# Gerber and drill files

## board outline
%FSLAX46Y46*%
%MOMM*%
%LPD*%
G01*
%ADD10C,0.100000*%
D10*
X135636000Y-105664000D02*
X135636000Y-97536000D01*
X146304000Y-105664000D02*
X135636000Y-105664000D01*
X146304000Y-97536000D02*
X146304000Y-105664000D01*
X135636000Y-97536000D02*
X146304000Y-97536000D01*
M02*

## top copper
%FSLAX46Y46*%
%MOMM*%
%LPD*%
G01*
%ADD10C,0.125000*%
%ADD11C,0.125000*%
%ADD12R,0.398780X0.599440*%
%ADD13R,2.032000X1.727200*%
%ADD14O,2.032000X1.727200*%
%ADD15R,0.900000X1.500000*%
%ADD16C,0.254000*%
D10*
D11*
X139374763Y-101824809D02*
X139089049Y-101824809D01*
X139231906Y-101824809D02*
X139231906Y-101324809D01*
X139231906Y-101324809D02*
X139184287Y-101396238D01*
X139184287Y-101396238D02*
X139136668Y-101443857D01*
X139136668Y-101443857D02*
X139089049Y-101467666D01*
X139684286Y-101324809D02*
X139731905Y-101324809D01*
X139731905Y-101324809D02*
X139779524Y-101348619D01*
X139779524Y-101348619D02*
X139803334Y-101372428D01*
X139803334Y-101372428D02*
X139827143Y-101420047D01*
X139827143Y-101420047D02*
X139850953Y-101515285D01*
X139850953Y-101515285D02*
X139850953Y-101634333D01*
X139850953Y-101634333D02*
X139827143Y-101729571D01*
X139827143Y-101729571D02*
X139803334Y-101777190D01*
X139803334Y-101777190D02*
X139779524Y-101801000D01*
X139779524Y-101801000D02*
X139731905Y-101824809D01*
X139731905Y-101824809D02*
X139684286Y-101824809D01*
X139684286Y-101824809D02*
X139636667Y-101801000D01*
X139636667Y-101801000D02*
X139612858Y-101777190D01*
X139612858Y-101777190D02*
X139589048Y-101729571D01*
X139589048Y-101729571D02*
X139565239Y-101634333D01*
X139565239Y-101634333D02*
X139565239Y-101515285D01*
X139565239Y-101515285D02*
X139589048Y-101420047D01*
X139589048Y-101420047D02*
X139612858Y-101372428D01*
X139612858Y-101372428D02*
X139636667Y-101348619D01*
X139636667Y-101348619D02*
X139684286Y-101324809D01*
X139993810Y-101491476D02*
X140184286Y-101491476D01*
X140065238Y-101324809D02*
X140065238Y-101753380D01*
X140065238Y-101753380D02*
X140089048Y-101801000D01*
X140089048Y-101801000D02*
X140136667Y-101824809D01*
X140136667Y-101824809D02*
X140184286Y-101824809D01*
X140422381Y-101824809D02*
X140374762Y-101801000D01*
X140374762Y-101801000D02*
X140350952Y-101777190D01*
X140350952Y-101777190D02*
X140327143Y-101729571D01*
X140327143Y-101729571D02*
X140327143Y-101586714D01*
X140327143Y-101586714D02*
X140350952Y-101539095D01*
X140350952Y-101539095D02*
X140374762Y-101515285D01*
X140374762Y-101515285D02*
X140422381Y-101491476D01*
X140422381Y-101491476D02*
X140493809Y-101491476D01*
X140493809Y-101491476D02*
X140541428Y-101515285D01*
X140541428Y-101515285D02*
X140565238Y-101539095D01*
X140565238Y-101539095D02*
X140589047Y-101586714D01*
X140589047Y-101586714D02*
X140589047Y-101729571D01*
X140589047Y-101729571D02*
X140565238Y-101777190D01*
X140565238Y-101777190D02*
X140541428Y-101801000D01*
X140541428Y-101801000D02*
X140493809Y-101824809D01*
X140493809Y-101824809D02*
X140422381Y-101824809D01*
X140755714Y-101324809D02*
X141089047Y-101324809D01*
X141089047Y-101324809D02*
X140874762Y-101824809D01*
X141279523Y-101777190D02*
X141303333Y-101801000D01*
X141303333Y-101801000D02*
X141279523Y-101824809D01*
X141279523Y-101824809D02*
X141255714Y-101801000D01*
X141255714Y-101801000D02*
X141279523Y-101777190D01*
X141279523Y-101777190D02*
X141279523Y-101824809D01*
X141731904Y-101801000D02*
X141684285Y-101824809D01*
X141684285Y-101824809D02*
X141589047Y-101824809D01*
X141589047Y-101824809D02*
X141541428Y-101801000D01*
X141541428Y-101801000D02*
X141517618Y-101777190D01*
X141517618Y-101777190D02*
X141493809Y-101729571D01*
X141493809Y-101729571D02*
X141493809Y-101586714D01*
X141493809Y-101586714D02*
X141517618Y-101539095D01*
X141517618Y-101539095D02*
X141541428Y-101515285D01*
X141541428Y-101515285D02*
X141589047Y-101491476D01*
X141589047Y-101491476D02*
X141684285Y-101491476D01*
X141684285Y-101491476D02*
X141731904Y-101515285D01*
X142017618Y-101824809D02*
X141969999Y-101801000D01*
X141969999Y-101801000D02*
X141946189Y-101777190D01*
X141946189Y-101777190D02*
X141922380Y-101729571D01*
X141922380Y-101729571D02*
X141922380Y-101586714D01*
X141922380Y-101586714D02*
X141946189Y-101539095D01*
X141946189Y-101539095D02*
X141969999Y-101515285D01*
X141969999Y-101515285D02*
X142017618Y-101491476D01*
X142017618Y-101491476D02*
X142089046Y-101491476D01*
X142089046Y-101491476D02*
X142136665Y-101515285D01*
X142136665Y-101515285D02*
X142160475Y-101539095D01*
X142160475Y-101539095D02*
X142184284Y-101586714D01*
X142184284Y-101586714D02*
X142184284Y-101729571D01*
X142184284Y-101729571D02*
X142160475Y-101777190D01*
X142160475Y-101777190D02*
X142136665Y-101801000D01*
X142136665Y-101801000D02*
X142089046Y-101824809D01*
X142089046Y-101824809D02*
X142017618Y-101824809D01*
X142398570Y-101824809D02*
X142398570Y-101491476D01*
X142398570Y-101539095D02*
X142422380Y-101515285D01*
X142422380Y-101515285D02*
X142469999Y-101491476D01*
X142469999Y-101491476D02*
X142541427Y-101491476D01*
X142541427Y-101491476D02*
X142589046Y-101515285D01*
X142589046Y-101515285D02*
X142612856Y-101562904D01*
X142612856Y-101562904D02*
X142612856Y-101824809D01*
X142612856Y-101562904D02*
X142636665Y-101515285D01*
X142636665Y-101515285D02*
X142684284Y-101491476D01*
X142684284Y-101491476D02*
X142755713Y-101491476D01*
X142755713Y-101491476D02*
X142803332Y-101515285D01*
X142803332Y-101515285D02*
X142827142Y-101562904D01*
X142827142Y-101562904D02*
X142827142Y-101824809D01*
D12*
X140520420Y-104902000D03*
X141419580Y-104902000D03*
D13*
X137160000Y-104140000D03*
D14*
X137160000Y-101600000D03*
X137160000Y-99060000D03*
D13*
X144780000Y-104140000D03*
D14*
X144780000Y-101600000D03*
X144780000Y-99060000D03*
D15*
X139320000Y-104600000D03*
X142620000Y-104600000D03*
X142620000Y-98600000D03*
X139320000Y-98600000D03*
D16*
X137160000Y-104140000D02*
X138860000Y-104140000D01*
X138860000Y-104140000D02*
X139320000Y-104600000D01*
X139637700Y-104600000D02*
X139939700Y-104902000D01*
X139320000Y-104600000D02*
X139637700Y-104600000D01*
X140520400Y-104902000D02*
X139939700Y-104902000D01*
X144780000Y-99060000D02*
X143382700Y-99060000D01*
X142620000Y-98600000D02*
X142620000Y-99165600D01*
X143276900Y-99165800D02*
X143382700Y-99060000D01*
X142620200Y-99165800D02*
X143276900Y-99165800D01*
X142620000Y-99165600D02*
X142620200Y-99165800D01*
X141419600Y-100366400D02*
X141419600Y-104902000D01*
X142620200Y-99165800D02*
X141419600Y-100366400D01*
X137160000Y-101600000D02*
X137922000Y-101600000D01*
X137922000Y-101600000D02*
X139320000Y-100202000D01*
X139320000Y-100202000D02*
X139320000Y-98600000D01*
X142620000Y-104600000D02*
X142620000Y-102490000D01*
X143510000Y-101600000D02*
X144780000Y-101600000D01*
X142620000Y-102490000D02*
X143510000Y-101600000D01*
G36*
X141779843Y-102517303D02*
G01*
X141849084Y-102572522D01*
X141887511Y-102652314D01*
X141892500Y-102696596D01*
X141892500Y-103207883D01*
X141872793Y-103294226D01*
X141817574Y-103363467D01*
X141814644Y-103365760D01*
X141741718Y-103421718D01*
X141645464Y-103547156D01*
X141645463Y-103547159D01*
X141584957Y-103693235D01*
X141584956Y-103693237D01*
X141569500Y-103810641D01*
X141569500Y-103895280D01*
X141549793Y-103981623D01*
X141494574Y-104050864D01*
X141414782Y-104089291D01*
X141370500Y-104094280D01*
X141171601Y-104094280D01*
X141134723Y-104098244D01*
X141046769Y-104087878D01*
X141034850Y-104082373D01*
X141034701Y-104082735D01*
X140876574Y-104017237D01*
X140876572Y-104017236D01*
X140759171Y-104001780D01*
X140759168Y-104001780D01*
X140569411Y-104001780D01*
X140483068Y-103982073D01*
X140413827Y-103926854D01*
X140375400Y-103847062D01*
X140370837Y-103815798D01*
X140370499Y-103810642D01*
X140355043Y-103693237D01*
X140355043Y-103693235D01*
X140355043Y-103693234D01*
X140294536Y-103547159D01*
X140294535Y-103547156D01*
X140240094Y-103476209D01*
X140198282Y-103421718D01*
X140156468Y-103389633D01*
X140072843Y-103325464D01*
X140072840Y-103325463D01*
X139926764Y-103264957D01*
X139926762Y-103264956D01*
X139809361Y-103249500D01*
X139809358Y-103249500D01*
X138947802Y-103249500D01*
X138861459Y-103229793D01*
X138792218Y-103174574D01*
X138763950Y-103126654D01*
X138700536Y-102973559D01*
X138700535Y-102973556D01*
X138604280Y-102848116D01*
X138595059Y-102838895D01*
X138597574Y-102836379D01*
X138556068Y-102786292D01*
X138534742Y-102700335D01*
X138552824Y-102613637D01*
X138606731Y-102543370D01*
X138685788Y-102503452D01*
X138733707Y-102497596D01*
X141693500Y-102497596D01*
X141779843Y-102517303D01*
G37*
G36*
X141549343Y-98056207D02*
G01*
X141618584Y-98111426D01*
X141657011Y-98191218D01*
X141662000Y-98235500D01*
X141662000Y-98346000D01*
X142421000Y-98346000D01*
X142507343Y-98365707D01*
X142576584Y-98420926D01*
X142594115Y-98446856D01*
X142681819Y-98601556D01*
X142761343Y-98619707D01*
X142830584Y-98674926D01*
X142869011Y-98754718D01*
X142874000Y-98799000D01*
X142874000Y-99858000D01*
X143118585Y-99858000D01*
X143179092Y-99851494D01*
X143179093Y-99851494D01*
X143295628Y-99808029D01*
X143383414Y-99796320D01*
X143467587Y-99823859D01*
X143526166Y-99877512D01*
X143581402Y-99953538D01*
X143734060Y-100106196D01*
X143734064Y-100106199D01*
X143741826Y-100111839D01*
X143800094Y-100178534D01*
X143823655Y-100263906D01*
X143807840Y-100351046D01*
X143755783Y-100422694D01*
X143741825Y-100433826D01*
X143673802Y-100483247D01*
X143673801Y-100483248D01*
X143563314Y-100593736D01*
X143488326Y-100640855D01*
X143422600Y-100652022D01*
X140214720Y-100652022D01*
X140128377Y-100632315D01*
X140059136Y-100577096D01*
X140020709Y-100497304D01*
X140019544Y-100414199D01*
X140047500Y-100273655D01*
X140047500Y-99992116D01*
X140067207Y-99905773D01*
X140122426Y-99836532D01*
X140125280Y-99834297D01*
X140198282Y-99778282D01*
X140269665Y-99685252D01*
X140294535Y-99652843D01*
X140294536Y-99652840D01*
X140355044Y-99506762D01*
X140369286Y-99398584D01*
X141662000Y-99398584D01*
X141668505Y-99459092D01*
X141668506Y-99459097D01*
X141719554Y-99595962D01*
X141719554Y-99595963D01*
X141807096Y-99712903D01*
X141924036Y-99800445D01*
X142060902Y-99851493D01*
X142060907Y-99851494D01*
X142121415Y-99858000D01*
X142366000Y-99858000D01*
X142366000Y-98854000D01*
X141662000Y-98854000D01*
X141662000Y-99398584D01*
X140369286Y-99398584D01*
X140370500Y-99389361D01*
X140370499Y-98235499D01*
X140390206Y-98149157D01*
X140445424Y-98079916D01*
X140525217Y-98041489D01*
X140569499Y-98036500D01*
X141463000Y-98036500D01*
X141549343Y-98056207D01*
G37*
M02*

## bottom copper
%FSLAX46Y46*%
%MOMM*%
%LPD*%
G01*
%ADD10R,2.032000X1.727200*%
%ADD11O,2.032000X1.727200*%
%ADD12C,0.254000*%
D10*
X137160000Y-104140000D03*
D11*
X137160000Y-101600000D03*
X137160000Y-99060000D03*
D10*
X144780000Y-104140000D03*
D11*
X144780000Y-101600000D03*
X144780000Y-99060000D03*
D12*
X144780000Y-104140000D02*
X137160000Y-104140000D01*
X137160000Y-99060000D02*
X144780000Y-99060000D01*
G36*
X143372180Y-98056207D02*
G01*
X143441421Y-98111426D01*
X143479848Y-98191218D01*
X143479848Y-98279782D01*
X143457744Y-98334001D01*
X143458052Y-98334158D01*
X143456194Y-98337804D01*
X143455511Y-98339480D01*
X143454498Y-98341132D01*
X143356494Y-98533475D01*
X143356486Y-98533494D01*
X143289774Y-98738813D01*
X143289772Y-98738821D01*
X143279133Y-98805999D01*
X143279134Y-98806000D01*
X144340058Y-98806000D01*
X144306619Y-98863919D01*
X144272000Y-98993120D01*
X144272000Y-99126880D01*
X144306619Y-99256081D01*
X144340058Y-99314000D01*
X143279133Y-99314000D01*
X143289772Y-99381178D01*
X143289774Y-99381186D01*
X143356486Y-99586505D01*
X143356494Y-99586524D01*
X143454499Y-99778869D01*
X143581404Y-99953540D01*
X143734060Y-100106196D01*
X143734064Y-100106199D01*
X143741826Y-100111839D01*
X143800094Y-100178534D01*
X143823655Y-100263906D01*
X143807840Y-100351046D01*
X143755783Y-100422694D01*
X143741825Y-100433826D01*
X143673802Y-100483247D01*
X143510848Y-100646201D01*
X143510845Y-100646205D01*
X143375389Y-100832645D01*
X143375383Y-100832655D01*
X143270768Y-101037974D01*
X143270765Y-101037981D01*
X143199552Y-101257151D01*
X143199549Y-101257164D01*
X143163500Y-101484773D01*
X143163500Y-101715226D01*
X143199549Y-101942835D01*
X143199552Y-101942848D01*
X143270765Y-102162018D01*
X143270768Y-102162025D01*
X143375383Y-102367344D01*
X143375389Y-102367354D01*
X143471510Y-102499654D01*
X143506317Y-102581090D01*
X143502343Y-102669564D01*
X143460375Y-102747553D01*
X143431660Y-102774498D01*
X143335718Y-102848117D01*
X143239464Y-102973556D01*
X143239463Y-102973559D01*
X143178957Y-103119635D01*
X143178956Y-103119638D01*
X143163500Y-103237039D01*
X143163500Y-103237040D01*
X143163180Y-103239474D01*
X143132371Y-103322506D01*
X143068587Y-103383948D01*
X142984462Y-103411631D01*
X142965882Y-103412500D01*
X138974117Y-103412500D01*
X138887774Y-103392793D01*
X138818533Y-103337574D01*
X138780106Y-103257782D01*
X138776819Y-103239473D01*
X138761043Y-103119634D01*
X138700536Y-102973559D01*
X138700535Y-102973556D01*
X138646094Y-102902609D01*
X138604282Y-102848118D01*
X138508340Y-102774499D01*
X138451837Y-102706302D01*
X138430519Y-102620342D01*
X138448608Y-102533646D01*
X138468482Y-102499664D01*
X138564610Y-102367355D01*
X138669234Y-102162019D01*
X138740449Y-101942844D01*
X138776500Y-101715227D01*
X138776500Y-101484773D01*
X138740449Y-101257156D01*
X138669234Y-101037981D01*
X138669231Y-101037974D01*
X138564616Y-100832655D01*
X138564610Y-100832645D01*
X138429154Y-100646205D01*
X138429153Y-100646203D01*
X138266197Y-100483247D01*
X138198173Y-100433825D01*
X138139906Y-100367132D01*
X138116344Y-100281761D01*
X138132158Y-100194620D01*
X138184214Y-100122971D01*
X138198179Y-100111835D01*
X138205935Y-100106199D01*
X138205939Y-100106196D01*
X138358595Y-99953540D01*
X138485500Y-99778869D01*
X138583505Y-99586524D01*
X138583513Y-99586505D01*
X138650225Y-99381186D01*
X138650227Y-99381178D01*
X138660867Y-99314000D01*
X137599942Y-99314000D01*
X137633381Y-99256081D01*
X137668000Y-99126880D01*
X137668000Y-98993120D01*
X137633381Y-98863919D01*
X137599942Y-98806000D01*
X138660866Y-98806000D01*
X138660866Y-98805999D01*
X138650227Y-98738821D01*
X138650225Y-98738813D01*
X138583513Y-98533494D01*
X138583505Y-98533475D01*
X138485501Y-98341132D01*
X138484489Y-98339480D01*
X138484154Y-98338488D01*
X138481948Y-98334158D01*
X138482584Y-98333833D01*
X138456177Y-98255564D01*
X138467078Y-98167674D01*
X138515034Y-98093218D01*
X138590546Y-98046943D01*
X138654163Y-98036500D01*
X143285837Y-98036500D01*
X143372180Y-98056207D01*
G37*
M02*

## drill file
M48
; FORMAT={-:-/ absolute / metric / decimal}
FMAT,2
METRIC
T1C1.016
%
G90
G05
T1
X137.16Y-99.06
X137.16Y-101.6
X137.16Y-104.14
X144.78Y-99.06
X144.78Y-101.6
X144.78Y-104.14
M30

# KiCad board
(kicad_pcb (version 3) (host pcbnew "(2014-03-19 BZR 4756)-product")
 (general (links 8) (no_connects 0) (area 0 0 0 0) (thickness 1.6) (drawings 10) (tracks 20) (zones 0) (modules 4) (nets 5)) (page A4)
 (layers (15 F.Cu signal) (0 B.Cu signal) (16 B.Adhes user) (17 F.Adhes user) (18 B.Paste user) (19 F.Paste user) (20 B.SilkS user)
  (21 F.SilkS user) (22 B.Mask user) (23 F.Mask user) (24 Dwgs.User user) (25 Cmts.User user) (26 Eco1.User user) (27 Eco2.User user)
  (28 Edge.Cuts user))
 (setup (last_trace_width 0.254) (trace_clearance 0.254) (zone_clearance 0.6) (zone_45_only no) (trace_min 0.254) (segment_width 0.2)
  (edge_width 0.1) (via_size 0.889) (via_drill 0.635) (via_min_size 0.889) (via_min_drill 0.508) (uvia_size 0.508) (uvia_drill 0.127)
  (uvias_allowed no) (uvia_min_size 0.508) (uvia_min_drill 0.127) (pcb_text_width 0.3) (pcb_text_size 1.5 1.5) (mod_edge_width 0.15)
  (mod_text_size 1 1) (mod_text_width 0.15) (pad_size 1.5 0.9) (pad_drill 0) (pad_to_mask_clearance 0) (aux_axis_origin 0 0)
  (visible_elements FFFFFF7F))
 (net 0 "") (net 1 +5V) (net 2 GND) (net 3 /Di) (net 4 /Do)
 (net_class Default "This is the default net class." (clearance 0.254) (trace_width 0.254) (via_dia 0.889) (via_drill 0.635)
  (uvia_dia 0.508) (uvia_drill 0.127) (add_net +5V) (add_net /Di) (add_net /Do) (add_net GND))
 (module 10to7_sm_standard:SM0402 (layer F.Cu) (at 140.97 104.902)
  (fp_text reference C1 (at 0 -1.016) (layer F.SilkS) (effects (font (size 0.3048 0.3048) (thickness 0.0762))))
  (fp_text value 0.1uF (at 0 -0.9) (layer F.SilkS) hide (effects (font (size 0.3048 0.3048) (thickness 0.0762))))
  (pad 1 smd rect (at -0.44958 0) (size 0.39878 0.59944) (layers F.Cu F.Paste F.Mask) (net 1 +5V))
  (pad 2 smd rect (at 0.44958 0) (size 0.39878 0.59944) (layers F.Cu F.Paste F.Mask) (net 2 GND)))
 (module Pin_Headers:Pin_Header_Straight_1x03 (layer F.Cu) (at 137.16 101.6 90)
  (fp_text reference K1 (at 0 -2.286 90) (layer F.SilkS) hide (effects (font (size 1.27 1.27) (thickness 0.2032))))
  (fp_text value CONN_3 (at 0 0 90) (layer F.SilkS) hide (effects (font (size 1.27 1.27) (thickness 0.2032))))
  (pad 1 thru_hole rect (at -2.54 0 90) (size 1.7272 2.032) (drill 1.016) (layers *.Cu *.Mask F.SilkS) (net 1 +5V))
  (pad 2 thru_hole oval (at 0 0 90) (size 1.7272 2.032) (drill 1.016) (layers *.Cu *.Mask F.SilkS) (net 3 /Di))
  (pad 3 thru_hole oval (at 2.54 0 90) (size 1.7272 2.032) (drill 1.016) (layers *.Cu *.Mask F.SilkS) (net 2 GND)))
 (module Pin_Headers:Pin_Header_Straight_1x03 (layer F.Cu) (at 144.78 101.6 90)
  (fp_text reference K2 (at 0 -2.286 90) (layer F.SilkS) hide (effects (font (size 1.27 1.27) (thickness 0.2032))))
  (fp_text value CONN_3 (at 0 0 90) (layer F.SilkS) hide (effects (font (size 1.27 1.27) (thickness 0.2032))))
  (pad 1 thru_hole rect (at -2.54 0 90) (size 1.7272 2.032) (drill 1.016) (layers *.Cu *.Mask F.SilkS) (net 1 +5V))
  (pad 2 thru_hole oval (at 0 0 90) (size 1.7272 2.032) (drill 1.016) (layers *.Cu *.Mask F.SilkS) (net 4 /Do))
  (pad 3 thru_hole oval (at 2.54 0 90) (size 1.7272 2.032) (drill 1.016) (layers *.Cu *.Mask F.SilkS) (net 2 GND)))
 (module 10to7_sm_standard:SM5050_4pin (layer F.Cu) (at 140.97 101.6 90)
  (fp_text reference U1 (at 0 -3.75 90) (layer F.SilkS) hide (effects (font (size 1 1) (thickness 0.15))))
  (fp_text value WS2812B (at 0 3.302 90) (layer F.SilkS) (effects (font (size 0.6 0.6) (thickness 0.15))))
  (pad 1 smd rect (at -3 -1.65 90) (size 1.5 0.9) (layers F.Cu F.Paste F.Mask) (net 1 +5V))
  (pad 2 smd rect (at -3 1.65 90) (size 1.5 0.9) (layers F.Cu F.Paste F.Mask) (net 4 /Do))
  (pad 3 smd rect (at 3 1.65 90) (size 1.5 0.9) (layers F.Cu F.Paste F.Mask) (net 2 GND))
  (pad 4 smd rect (at 3 -1.65 90) (size 1.5 0.9) (layers F.Cu F.Paste F.Mask) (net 3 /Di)))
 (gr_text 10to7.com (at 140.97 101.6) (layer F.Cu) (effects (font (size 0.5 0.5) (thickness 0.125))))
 (gr_line (start 135.636 105.664) (end 135.636 97.536) (angle 90) (layer Edge.Cuts) (width 0.1))
 (gr_line (start 146.304 105.664) (end 135.636 105.664) (angle 90) (layer Edge.Cuts) (width 0.1))
 (gr_line (start 146.304 97.536) (end 146.304 105.664) (angle 90) (layer Edge.Cuts) (width 0.1))
 (gr_line (start 135.636 97.536) (end 146.304 97.536) (angle 90) (layer Edge.Cuts) (width 0.1))
 (segment (start 137.16 104.14) (end 138.86 104.14) (width 0.254) (layer F.Cu) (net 1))
 (segment (start 138.86 104.14) (end 139.32 104.6) (width 0.254) (layer F.Cu) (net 1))
 (segment (start 139.6377 104.6) (end 139.9397 104.902) (width 0.254) (layer F.Cu) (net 1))
 (segment (start 139.32 104.6) (end 139.6377 104.6) (width 0.254) (layer F.Cu) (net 1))
 (segment (start 140.5204 104.902) (end 139.9397 104.902) (width 0.254) (layer F.Cu) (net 1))
 (segment (start 144.78 104.14) (end 137.16 104.14) (width 0.254) (layer B.Cu) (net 1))
 (segment (start 144.78 99.06) (end 143.3827 99.06) (width 0.254) (layer F.Cu) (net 2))
 (segment (start 142.62 98.6) (end 142.62 99.1656) (width 0.254) (layer F.Cu) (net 2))
 (segment (start 143.2769 99.1658) (end 143.3827 99.06) (width 0.254) (layer F.Cu) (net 2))
 (segment (start 142.6202 99.1658) (end 143.2769 99.1658) (width 0.254) (layer F.Cu) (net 2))
 (segment (start 142.62 99.1656) (end 142.6202 99.1658) (width 0.254) (layer F.Cu) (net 2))
 (segment (start 141.4196 100.3664) (end 141.4196 104.902) (width 0.254) (layer F.Cu) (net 2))
 (segment (start 142.6202 99.1658) (end 141.4196 100.3664) (width 0.254) (layer F.Cu) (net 2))
 (segment (start 137.16 99.06) (end 144.78 99.06) (width 0.254) (layer B.Cu) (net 2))
 (segment (start 137.16 101.6) (end 137.922 101.6) (width 0.254) (layer F.Cu) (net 3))
 (segment (start 137.922 101.6) (end 139.32 100.202) (width 0.254) (layer F.Cu) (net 3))
 (segment (start 139.32 100.202) (end 139.32 98.6) (width 0.254) (layer F.Cu) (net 3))
 (segment (start 142.62 104.6) (end 142.62 102.49) (width 0.254) (layer F.Cu) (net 4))
 (segment (start 143.51 101.6) (end 144.78 101.6) (width 0.254) (layer F.Cu) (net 4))
 (segment (start 142.62 102.49) (end 143.51 101.6) (width 0.254) (layer F.Cu) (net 4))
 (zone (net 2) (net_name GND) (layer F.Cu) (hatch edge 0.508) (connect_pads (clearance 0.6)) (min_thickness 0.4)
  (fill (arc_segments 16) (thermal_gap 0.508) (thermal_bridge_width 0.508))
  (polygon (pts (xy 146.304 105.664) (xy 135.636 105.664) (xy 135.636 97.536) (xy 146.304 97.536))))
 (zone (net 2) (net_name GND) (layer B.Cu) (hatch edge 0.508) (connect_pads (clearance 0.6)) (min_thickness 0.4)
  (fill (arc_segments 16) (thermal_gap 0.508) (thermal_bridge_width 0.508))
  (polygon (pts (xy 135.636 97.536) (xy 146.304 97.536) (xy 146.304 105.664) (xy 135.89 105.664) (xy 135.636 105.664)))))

